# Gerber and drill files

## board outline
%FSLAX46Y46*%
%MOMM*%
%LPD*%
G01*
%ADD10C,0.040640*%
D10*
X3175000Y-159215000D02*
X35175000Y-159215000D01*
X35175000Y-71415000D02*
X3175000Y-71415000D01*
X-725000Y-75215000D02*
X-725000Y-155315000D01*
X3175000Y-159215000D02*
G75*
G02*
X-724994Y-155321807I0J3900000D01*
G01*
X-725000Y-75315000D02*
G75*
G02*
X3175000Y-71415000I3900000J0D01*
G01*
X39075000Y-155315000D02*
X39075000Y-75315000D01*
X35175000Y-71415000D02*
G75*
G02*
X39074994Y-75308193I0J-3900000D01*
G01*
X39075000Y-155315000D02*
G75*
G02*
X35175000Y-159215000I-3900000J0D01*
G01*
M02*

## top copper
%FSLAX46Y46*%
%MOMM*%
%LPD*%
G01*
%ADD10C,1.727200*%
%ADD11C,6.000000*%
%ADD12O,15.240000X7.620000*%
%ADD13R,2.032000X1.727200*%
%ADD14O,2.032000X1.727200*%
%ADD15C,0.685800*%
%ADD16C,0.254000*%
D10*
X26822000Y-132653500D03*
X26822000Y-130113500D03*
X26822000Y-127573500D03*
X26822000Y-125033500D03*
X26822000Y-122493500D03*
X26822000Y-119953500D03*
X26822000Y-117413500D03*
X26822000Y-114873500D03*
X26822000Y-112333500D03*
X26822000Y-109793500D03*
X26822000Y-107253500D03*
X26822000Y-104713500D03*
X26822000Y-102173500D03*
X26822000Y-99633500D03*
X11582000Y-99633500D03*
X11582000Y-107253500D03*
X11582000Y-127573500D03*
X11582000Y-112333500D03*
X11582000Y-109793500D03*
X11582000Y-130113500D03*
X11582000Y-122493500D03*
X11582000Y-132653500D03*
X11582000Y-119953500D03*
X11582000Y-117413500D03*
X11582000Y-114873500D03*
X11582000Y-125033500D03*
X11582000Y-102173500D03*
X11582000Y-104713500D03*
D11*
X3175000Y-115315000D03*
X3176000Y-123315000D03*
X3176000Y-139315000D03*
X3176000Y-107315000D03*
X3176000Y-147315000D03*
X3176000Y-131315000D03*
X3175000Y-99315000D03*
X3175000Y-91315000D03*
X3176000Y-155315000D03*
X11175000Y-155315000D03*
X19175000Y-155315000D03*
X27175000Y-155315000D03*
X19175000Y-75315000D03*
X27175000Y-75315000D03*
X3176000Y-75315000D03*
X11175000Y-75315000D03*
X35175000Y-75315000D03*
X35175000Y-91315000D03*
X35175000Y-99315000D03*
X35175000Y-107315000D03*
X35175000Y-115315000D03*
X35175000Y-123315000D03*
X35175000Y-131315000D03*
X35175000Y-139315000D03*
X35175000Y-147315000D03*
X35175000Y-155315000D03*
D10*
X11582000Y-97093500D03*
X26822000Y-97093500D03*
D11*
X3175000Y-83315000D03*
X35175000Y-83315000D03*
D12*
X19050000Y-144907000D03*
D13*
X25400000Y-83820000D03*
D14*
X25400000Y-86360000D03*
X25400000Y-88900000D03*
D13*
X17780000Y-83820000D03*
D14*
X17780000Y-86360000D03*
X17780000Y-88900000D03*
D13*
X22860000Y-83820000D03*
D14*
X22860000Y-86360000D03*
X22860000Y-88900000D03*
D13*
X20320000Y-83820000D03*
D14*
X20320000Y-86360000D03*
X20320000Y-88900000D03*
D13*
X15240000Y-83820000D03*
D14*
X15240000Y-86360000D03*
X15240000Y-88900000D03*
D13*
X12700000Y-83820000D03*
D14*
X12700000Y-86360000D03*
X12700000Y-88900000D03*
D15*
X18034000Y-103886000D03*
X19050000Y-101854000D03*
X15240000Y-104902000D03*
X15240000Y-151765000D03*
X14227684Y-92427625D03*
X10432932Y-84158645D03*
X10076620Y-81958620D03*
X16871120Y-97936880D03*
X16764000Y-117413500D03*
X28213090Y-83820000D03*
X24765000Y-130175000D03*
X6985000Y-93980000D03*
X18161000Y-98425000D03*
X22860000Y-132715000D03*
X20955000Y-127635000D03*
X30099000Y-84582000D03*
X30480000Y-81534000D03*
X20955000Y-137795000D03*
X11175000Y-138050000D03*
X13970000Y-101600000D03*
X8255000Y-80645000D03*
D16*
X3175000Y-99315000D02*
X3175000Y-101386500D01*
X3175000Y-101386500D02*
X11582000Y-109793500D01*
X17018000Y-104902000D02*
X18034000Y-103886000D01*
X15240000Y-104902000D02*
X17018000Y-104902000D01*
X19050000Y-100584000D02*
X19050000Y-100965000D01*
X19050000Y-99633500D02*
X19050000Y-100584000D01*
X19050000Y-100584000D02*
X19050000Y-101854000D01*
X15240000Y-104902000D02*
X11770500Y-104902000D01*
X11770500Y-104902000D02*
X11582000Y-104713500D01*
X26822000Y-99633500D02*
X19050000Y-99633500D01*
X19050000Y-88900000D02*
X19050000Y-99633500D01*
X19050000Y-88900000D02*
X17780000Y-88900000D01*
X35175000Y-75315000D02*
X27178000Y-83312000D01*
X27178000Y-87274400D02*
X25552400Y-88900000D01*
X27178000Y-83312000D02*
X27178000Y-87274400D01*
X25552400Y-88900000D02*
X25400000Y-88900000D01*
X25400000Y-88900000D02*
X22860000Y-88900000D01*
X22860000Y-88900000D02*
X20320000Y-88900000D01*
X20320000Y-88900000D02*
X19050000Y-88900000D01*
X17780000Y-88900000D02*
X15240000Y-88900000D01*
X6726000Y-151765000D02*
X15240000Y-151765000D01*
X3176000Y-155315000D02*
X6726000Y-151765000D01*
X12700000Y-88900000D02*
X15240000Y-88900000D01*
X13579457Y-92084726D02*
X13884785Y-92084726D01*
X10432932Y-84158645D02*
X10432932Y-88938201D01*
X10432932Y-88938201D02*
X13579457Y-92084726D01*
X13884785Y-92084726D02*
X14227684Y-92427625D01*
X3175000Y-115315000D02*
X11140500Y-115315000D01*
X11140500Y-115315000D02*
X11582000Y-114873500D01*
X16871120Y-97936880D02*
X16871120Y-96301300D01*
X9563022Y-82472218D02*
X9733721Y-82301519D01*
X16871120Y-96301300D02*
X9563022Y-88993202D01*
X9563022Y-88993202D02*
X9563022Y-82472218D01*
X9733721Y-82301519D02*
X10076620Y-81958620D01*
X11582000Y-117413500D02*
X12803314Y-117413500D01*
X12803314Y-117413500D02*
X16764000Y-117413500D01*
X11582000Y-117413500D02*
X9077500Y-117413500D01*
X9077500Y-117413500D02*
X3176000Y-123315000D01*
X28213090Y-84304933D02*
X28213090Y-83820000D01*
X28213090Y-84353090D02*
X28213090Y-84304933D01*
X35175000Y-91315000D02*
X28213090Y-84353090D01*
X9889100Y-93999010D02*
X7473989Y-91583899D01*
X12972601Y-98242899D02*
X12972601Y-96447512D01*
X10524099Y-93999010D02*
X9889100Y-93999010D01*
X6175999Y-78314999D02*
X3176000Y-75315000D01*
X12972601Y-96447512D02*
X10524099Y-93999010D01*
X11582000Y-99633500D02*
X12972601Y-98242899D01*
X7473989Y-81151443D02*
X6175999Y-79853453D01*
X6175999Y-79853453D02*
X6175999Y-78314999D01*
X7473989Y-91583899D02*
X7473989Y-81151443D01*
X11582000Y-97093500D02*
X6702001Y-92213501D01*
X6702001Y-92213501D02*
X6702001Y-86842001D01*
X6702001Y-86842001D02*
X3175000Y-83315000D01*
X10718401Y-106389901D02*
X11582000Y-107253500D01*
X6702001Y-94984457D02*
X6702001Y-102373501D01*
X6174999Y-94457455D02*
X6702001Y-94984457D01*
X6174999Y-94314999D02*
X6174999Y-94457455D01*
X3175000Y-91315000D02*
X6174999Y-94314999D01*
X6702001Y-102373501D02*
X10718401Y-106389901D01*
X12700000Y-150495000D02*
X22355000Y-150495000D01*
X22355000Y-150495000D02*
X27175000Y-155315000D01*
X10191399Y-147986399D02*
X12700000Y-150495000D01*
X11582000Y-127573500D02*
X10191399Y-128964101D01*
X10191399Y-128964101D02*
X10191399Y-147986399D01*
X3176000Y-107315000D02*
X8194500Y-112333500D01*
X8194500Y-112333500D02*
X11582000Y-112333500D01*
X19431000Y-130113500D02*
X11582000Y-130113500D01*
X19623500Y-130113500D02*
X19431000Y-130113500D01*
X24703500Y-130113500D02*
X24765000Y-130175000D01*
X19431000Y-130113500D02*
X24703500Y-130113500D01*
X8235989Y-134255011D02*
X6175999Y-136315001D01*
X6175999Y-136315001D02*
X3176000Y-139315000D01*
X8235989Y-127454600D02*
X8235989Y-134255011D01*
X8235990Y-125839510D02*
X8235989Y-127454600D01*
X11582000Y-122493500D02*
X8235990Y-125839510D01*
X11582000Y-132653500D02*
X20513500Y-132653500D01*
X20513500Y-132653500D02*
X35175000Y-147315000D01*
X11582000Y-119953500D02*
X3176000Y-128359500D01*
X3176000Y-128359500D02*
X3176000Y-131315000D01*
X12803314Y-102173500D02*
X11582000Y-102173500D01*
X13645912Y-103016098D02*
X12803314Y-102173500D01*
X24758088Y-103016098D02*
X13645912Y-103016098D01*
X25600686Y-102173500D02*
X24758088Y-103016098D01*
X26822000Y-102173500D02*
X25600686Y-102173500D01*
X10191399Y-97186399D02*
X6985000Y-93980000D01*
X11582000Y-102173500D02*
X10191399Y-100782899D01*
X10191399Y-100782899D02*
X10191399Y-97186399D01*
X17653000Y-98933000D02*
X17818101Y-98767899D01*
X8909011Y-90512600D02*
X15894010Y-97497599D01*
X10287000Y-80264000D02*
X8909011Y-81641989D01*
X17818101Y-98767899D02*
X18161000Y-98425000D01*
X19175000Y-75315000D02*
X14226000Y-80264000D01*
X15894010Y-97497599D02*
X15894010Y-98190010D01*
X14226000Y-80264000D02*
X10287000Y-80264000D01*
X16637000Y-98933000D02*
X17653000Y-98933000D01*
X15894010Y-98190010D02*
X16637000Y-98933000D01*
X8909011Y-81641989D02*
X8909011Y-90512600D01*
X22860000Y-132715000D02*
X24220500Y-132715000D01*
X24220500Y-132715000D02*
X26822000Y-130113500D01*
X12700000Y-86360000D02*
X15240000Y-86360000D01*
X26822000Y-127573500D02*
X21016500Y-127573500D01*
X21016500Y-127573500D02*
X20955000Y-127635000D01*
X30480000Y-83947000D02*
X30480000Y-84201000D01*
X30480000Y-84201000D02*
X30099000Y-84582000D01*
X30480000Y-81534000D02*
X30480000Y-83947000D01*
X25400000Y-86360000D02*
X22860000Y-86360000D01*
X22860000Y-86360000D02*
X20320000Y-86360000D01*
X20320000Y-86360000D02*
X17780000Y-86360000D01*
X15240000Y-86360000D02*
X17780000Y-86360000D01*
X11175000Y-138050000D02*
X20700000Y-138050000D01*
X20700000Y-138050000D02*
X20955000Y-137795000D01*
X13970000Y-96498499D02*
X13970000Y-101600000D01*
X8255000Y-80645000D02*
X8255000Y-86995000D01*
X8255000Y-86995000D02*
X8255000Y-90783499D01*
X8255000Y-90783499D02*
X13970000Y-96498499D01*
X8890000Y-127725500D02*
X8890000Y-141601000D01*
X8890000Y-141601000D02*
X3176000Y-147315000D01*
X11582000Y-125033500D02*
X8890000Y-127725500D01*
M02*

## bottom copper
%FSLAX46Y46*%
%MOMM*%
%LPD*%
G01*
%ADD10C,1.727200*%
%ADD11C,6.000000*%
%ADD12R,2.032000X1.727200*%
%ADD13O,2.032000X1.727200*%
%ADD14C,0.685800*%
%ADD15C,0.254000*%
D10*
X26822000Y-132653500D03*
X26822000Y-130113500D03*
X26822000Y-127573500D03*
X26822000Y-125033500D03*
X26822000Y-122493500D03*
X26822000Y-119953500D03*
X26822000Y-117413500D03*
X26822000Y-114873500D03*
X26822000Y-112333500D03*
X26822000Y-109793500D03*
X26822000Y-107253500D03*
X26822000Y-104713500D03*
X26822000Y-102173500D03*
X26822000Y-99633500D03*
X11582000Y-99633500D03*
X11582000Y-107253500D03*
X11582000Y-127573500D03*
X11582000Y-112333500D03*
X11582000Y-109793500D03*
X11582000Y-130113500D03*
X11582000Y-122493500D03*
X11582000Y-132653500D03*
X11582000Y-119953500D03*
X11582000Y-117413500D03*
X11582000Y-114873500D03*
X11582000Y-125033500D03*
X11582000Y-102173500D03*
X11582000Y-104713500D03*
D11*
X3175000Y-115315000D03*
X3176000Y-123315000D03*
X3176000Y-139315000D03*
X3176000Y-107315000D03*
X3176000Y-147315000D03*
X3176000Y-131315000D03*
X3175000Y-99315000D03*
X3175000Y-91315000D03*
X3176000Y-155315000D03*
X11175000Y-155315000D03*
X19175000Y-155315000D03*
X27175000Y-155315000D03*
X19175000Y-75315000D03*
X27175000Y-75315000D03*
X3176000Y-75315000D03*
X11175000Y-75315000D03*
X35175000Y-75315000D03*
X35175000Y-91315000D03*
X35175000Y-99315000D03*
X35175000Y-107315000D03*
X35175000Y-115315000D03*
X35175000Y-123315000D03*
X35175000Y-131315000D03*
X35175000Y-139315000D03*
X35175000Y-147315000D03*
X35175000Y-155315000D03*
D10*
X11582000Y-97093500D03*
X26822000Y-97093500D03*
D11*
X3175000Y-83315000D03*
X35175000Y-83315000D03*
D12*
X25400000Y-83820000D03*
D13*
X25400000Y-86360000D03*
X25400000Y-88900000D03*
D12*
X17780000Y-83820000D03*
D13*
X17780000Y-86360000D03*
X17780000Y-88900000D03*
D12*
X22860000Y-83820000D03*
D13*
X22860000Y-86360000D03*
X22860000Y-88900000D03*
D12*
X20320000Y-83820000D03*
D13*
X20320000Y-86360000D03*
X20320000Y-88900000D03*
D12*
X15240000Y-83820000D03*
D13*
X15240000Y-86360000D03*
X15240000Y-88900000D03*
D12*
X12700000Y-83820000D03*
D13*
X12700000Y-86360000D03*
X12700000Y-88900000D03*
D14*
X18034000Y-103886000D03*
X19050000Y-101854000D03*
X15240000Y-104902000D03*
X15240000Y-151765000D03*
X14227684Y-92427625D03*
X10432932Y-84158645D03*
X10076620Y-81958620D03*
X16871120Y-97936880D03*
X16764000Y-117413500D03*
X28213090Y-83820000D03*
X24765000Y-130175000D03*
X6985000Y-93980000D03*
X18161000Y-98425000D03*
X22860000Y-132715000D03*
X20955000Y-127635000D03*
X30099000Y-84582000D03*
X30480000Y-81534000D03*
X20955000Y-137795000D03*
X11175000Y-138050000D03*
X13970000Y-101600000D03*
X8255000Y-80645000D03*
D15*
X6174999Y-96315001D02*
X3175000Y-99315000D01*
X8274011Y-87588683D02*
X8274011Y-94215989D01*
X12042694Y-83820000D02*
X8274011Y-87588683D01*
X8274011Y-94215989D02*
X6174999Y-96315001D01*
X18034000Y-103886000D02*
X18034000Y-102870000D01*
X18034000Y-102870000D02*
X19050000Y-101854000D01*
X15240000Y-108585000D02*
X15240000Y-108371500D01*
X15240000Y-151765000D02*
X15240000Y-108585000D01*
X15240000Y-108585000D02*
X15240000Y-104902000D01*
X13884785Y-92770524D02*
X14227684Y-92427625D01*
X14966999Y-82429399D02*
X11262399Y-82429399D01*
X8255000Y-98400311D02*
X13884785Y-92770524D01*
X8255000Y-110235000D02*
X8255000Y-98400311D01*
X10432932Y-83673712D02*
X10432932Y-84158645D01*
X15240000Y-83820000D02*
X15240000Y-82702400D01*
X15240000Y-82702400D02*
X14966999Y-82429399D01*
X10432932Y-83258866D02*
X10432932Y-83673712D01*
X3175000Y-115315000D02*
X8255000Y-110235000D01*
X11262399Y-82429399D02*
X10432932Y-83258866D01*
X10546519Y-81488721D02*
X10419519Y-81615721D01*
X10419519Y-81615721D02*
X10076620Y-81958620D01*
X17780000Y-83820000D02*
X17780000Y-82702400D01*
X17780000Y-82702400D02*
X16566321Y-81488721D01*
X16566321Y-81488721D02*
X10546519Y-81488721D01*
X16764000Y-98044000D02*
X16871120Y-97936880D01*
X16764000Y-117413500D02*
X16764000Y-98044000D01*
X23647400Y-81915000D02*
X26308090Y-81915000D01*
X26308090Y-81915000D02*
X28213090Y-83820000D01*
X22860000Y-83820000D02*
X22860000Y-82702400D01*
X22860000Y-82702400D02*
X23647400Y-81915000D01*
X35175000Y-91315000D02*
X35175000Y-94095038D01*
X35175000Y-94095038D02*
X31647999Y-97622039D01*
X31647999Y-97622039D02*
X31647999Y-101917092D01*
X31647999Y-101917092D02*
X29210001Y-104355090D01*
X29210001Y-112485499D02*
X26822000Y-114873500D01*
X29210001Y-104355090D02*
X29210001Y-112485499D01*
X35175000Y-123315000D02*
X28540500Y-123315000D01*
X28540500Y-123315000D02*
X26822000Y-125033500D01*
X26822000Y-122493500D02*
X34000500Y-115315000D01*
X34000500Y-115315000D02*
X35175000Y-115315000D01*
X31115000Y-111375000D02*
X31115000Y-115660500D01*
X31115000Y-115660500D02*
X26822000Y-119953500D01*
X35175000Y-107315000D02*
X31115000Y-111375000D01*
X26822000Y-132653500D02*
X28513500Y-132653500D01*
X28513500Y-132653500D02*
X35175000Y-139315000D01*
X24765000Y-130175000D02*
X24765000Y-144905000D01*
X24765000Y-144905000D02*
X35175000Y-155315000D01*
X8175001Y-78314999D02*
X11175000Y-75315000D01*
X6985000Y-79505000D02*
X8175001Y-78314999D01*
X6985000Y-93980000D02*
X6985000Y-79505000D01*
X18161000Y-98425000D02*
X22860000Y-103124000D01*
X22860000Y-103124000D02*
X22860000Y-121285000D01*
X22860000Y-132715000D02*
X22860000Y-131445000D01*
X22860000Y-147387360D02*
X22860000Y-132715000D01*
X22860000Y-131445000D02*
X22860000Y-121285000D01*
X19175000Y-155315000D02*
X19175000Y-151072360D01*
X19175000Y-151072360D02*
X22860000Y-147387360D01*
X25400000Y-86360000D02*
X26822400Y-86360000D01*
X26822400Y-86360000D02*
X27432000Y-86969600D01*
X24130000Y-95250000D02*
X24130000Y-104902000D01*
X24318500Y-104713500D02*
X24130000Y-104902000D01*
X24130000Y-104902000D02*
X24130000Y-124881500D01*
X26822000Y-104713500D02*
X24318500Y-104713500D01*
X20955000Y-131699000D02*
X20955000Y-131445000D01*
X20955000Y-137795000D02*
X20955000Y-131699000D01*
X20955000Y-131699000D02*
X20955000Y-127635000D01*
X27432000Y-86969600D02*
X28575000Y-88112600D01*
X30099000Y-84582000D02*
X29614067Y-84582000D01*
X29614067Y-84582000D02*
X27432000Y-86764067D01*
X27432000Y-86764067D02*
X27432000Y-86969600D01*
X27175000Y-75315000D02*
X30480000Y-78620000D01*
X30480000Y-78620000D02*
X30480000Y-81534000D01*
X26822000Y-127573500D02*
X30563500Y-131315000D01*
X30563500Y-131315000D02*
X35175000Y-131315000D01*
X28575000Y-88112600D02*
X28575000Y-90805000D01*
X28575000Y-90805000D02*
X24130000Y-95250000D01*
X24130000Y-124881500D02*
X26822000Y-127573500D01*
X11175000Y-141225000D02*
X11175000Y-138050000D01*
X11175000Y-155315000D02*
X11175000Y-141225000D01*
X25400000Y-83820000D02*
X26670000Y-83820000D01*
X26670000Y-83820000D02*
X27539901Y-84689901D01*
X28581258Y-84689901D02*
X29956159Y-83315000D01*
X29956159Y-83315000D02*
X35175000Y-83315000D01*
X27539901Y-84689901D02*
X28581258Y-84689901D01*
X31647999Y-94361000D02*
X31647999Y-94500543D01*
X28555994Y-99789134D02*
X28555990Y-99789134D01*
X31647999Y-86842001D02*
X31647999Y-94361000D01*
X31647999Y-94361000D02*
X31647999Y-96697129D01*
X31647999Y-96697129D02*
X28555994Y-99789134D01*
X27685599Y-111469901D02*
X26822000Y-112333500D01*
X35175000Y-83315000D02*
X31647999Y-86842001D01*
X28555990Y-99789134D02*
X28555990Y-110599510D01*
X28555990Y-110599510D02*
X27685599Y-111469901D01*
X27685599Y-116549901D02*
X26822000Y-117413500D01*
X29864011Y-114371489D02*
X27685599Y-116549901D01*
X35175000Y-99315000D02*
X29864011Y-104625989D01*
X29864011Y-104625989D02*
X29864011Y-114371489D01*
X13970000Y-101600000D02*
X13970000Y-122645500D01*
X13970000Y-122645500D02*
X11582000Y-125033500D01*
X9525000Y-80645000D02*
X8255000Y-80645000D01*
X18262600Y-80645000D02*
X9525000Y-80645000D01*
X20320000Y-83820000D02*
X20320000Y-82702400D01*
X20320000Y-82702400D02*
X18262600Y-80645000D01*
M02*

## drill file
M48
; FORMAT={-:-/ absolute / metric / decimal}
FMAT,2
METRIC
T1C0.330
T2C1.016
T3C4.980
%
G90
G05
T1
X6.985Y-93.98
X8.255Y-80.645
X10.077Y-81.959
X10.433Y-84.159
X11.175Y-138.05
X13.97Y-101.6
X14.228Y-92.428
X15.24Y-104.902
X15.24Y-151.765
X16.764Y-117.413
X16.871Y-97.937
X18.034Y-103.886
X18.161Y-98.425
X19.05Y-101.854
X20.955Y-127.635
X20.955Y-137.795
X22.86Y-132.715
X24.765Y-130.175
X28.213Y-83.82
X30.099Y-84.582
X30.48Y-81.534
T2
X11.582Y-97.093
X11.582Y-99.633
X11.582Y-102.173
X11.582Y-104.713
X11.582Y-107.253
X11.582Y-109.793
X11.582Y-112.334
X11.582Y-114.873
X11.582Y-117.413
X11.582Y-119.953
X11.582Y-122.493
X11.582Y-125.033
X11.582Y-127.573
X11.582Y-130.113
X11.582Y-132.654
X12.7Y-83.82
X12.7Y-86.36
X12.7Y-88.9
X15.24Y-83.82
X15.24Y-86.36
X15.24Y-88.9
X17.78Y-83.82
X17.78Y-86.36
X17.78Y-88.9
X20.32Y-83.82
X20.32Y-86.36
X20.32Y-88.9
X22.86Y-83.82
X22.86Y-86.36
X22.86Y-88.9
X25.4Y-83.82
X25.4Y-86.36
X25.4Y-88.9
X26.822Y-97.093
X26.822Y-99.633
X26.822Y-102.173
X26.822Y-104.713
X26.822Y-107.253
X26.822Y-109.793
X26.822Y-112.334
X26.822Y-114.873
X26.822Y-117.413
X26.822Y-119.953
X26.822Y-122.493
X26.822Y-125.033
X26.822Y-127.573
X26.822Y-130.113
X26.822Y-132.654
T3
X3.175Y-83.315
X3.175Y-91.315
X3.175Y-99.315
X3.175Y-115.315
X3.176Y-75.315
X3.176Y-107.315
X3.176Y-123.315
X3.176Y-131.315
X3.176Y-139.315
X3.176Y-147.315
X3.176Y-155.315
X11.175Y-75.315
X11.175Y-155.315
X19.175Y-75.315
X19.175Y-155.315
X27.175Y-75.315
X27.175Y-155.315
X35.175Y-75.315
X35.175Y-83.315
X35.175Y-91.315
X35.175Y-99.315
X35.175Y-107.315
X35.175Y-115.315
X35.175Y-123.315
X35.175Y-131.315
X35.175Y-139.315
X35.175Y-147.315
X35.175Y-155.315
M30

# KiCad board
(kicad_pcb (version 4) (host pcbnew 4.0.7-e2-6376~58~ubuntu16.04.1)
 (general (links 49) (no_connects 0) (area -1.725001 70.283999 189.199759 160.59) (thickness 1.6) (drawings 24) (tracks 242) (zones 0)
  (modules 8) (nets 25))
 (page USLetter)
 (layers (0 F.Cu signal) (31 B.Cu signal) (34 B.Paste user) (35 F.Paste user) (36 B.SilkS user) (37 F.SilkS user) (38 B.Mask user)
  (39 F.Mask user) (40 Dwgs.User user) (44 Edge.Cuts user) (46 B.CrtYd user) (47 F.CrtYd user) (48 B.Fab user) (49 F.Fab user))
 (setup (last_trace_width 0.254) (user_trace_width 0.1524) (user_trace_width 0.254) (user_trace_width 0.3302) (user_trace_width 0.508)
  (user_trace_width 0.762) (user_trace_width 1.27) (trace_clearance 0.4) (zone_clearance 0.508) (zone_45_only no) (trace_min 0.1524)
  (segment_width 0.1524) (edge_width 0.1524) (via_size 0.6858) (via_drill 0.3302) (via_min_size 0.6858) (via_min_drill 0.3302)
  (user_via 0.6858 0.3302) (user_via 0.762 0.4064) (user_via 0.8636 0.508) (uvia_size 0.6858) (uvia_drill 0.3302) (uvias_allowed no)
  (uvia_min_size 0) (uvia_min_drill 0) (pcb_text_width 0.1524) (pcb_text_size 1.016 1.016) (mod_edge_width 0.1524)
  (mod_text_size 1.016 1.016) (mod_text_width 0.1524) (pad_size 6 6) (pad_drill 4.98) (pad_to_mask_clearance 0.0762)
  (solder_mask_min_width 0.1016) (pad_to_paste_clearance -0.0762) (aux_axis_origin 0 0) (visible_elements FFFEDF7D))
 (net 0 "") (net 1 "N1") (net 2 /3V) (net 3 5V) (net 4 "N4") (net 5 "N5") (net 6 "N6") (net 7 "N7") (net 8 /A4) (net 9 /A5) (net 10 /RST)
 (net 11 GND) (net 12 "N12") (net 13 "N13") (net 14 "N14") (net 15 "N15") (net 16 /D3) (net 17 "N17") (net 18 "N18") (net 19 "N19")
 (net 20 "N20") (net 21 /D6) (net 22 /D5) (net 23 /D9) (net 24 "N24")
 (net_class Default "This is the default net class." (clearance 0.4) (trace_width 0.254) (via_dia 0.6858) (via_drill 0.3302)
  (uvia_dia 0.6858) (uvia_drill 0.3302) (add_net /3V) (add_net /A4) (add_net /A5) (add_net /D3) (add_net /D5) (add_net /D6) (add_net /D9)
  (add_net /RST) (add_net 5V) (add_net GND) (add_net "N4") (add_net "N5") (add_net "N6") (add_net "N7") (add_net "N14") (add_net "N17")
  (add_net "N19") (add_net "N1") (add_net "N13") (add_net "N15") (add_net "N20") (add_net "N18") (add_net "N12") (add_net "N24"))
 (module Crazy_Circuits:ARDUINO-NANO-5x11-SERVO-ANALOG (layer F.Cu) (at 3.175 107.315)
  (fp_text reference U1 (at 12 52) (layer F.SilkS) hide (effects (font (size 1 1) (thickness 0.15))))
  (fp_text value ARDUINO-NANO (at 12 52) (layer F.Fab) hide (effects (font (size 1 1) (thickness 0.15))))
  (fp_line (start 0 51.9) (end 32 51.9) (layer Edge.Cuts) (width 0.04064))
  (fp_line (start 32 -35.9) (end 0 -35.9) (layer Edge.Cuts) (width 0.04064))
  (fp_line (start -3.9 -32.1) (end -3.9 48) (layer Edge.Cuts) (width 0.04064))
  (fp_arc (start 0 48) (end 0 51.9) (angle 89.9) (layer Edge.Cuts) (width 0.04064))
  (fp_arc (start 0 -32) (end -3.9 -32) (angle 90) (layer Edge.Cuts) (width 0.04064))
  (fp_line (start 35.9 48) (end 35.9 -32) (layer Edge.Cuts) (width 0.04064))
  (fp_arc (start 32 -32) (end 32 -35.9) (angle 89.9) (layer Edge.Cuts) (width 0.04064))
  (fp_arc (start 32 48) (end 35.9 48) (angle 90) (layer Edge.Cuts) (width 0.04064))
  (pad D13 thru_hole circle (at 23.647 25.3385 180) (size 1.7272 1.7272) (drill 1.016) (layers *.Cu *.Mask F.SilkS) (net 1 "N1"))
  (pad 3V thru_hole circle (at 23.647 22.7985 180) (size 1.7272 1.7272) (drill 1.016) (layers *.Cu *.Mask F.SilkS) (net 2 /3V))
  (pad REF thru_hole circle (at 23.647 20.2585 180) (size 1.7272 1.7272) (drill 1.016) (layers *.Cu *.Mask F.SilkS) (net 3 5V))
  (pad A0 thru_hole circle (at 23.647 17.7185 180) (size 1.7272 1.7272) (drill 1.016) (layers *.Cu *.Mask F.SilkS) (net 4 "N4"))
  (pad A1 thru_hole circle (at 23.647 15.1785 180) (size 1.7272 1.7272) (drill 1.016) (layers *.Cu *.Mask F.SilkS) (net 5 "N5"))
  (pad A2 thru_hole circle (at 23.647 12.6385 180) (size 1.7272 1.7272) (drill 1.016) (layers *.Cu *.Mask F.SilkS) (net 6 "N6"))
  (pad A3 thru_hole circle (at 23.647 10.0985 180) (size 1.7272 1.7272) (drill 1.016) (layers *.Cu *.Mask F.SilkS) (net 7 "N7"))
  (pad A4 thru_hole circle (at 23.647 7.5585 180) (size 1.7272 1.7272) (drill 1.016) (layers *.Cu *.Mask F.SilkS) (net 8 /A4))
  (pad A5 thru_hole circle (at 23.647 5.0185 180) (size 1.7272 1.7272) (drill 1.016) (layers *.Cu *.Mask F.SilkS) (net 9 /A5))
  (pad A6 thru_hole circle (at 23.647 2.4785 180) (size 1.7272 1.7272) (drill 1.016) (layers *.Cu *.Mask F.SilkS))
  (pad A7 thru_hole circle (at 23.647 -0.0615 180) (size 1.7272 1.7272) (drill 1.016) (layers *.Cu *.Mask F.SilkS))
  (pad 5V thru_hole circle (at 23.647 -2.6015 180) (size 1.7272 1.7272) (drill 1.016) (layers *.Cu *.Mask F.SilkS) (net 3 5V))
  (pad RST thru_hole circle (at 23.647 -5.1415 180) (size 1.7272 1.7272) (drill 1.016) (layers *.Cu *.Mask F.SilkS) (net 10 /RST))
  (pad GND thru_hole circle (at 23.647 -7.6815 180) (size 1.7272 1.7272) (drill 1.016) (layers *.Cu *.Mask F.SilkS) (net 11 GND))
  (pad RX0 thru_hole circle (at 8.407 -7.6815 180) (size 1.7272 1.7272) (drill 1.016) (layers *.Cu *.Mask F.SilkS) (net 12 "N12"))
  (pad D2 thru_hole circle (at 8.407 -0.0615 180) (size 1.7272 1.7272) (drill 1.016) (layers *.Cu *.Mask F.SilkS) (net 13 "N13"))
  (pad D10 thru_hole circle (at 8.407 20.2585 180) (size 1.7272 1.7272) (drill 1.016) (layers *.Cu *.Mask F.SilkS) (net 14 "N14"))
  (pad D4 thru_hole circle (at 8.407 5.0185 180) (size 1.7272 1.7272) (drill 1.016) (layers *.Cu *.Mask F.SilkS) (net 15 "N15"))
  (pad D3 thru_hole circle (at 8.407 2.4785 180) (size 1.7272 1.7272) (drill 1.016) (layers *.Cu *.Mask F.SilkS) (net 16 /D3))
  (pad D11 thru_hole circle (at 8.407 22.7985 180) (size 1.7272 1.7272) (drill 1.016) (layers *.Cu *.Mask F.SilkS) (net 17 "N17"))
  (pad D8 thru_hole circle (at 8.407 15.1785 180) (size 1.7272 1.7272) (drill 1.016) (layers *.Cu *.Mask F.SilkS) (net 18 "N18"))
  (pad D12 thru_hole circle (at 8.407 25.3385 180) (size 1.7272 1.7272) (drill 1.016) (layers *.Cu *.Mask F.SilkS) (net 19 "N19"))
  (pad D7 thru_hole circle (at 8.407 12.6385 180) (size 1.7272 1.7272) (drill 1.016) (layers *.Cu *.Mask F.SilkS) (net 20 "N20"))
  (pad D6 thru_hole circle (at 8.407 10.0985 180) (size 1.7272 1.7272) (drill 1.016) (layers *.Cu *.Mask F.SilkS) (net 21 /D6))
  (pad D5 thru_hole circle (at 8.407 7.5585 180) (size 1.7272 1.7272) (drill 1.016) (layers *.Cu *.Mask F.SilkS) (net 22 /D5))
  (pad D9 thru_hole circle (at 8.407 17.7185 180) (size 1.7272 1.7272) (drill 1.016) (layers *.Cu *.Mask F.SilkS) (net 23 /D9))
  (pad RST thru_hole circle (at 8.407 -5.1415 180) (size 1.7272 1.7272) (drill 1.016) (layers *.Cu *.Mask F.SilkS) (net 10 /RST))
  (pad GND thru_hole circle (at 8.407 -2.6015 180) (size 1.7272 1.7272) (drill 1.016) (layers *.Cu *.Mask F.SilkS) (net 11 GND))
  (pad D5 thru_hole circle (at 0 8 90) (size 6 6) (drill 4.98) (layers *.Cu *.Mask) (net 22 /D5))
  (pad D6 thru_hole circle (at 0.001 16 90) (size 6 6) (drill 4.98) (layers *.Cu *.Mask) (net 21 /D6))
  (pad D8 thru_hole circle (at 0.001 32 90) (size 6 6) (drill 4.98) (layers *.Cu *.Mask) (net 18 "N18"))
  (pad D4 thru_hole circle (at 0.001 0 90) (size 6 6) (drill 4.98) (layers *.Cu *.Mask) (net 15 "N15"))
  (pad D9 thru_hole circle (at 0.001 40 90) (size 6 6) (drill 4.98) (layers *.Cu *.Mask) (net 23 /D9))
  (pad D7 thru_hole circle (at 0.001 24 90) (size 6 6) (drill 4.98) (layers *.Cu *.Mask) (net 20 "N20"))
  (pad D3 thru_hole circle (at 0 -8 90) (size 6 6) (drill 4.98) (layers *.Cu *.Mask) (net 16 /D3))
  (pad D2 thru_hole circle (at 0 -16 90) (size 6 6) (drill 4.98) (layers *.Cu *.Mask) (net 13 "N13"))
  (pad GND thru_hole circle (at 0.001 48 90) (size 6 6) (drill 4.98) (layers *.Cu *.Mask) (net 11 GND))
  (pad 5V thru_hole circle (at 8 48 90) (size 6 6) (drill 4.98) (layers *.Cu *.Mask) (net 3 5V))
  (pad 3V thru_hole circle (at 16 48 90) (size 6 6) (drill 4.98) (layers *.Cu *.Mask) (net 2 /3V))
  (pad D10 thru_hole circle (at 24 48 90) (size 6 6) (drill 4.98) (layers *.Cu *.Mask) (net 14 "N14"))
  (pad 3V thru_hole circle (at 16 -32 90) (size 6 6) (drill 4.98) (layers *.Cu *.Mask) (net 2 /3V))
  (pad 5V thru_hole circle (at 24 -32 90) (size 6 6) (drill 4.98) (layers *.Cu *.Mask) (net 3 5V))
  (pad RX0 thru_hole circle (at 0.001 -32 90) (size 6 6) (drill 4.98) (layers *.Cu *.Mask) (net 12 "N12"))
  (pad RST thru_hole circle (at 8 -32 90) (size 6 6) (drill 4.98) (layers *.Cu *.Mask) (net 10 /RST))
  (pad GND thru_hole circle (at 32 -32 90) (size 6 6) (drill 4.98) (layers *.Cu *.Mask) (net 11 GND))
  (pad A4 thru_hole circle (at 32 -16 90) (size 6 6) (drill 4.98) (layers *.Cu *.Mask) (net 8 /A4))
  (pad A3 thru_hole circle (at 32 -8 90) (size 6 6) (drill 4.98) (layers *.Cu *.Mask) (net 7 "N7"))
  (pad A2 thru_hole circle (at 32 0 90) (size 6 6) (drill 4.98) (layers *.Cu *.Mask) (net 6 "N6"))
  (pad A1 thru_hole circle (at 32 8 90) (size 6 6) (drill 4.98) (layers *.Cu *.Mask) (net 5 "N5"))
  (pad A0 thru_hole circle (at 32 16 90) (size 6 6) (drill 4.98) (layers *.Cu *.Mask) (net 4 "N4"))
  (pad REF thru_hole circle (at 32 24 90) (size 6 6) (drill 4.98) (layers *.Cu *.Mask) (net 3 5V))
  (pad D13 thru_hole circle (at 32 32 90) (size 6 6) (drill 4.98) (layers *.Cu *.Mask) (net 1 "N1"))
  (pad D12 thru_hole circle (at 32 40 90) (size 6 6) (drill 4.98) (layers *.Cu *.Mask) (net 19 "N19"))
  (pad D11 thru_hole circle (at 32 48 90) (size 6 6) (drill 4.98) (layers *.Cu *.Mask) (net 17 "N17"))
  (pad TX1 thru_hole circle (at 8.407 -10.2215 180) (size 1.7272 1.7272) (drill 1.016) (layers *.Cu *.Mask F.SilkS) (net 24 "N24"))
  (pad VIN thru_hole circle (at 23.647 -10.2215 180) (size 1.7272 1.7272) (drill 1.016) (layers *.Cu *.Mask F.SilkS))
  (pad TX1 thru_hole circle (at 0 -24 90) (size 6 6) (drill 4.98) (layers *.Cu *.Mask) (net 24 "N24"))
  (pad A5 thru_hole circle (at 32 -24 90) (size 6 6) (drill 4.98) (layers *.Cu *.Mask) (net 9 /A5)))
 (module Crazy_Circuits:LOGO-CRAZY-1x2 (layer F.Cu) (at 19.05 148.844)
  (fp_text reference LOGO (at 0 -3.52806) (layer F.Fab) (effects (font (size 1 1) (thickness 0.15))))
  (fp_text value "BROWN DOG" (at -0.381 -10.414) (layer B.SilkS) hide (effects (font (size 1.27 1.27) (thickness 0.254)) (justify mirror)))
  (pad BG smd oval (at 0 -3.937) (size 15.24 7.62) (layers F.Cu)))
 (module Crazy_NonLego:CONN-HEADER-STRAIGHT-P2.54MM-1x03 (layer F.Cu) (at 25.4 83.82)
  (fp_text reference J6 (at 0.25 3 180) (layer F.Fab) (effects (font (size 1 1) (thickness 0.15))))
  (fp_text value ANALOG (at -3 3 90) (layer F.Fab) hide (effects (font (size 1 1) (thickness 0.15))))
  (pad 1 thru_hole rect (at 0 0) (size 2.032 1.7272) (drill 1.016) (layers *.Cu *.Mask F.SilkS) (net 9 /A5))
  (pad 2 thru_hole oval (at 0 2.54) (size 2.032 1.7272) (drill 1.016) (layers *.Cu *.Mask F.SilkS) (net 3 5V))
  (pad 3 thru_hole oval (at 0 5.08) (size 2.032 1.7272) (drill 1.016) (layers *.Cu *.Mask F.SilkS) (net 11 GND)))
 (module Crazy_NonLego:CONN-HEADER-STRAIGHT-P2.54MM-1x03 (layer F.Cu) (at 17.78 83.82)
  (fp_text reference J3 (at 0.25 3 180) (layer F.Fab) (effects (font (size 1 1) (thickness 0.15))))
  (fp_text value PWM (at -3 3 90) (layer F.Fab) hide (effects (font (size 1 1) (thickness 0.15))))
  (pad 1 thru_hole rect (at 0 0) (size 2.032 1.7272) (drill 1.016) (layers *.Cu *.Mask F.SilkS) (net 21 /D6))
  (pad 2 thru_hole oval (at 0 2.54) (size 2.032 1.7272) (drill 1.016) (layers *.Cu *.Mask F.SilkS) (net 3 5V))
  (pad 3 thru_hole oval (at 0 5.08) (size 2.032 1.7272) (drill 1.016) (layers *.Cu *.Mask F.SilkS) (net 11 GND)))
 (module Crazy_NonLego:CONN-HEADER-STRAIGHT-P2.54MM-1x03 (layer F.Cu) (at 22.86 83.82)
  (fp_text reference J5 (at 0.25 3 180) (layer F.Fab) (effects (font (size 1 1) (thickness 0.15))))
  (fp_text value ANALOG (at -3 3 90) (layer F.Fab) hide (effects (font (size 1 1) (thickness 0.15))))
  (pad 1 thru_hole rect (at 0 0) (size 2.032 1.7272) (drill 1.016) (layers *.Cu *.Mask F.SilkS) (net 8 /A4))
  (pad 2 thru_hole oval (at 0 2.54) (size 2.032 1.7272) (drill 1.016) (layers *.Cu *.Mask F.SilkS) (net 3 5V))
  (pad 3 thru_hole oval (at 0 5.08) (size 2.032 1.7272) (drill 1.016) (layers *.Cu *.Mask F.SilkS) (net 11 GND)))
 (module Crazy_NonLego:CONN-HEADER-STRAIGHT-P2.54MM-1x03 (layer F.Cu) (at 20.32 83.82)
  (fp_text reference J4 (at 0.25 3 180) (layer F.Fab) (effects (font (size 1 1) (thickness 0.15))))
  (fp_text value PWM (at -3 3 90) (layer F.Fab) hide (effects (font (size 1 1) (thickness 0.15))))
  (pad 1 thru_hole rect (at 0 0) (size 2.032 1.7272) (drill 1.016) (layers *.Cu *.Mask F.SilkS) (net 23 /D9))
  (pad 2 thru_hole oval (at 0 2.54) (size 2.032 1.7272) (drill 1.016) (layers *.Cu *.Mask F.SilkS) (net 3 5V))
  (pad 3 thru_hole oval (at 0 5.08) (size 2.032 1.7272) (drill 1.016) (layers *.Cu *.Mask F.SilkS) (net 11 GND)))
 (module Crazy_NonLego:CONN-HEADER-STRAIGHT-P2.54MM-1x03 (layer F.Cu) (at 15.24 83.82)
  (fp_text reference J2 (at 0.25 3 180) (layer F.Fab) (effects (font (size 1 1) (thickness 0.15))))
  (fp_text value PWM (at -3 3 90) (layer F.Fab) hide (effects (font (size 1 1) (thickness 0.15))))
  (pad 1 thru_hole rect (at 0 0) (size 2.032 1.7272) (drill 1.016) (layers *.Cu *.Mask F.SilkS) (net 22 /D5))
  (pad 2 thru_hole oval (at 0 2.54) (size 2.032 1.7272) (drill 1.016) (layers *.Cu *.Mask F.SilkS) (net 3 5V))
  (pad 3 thru_hole oval (at 0 5.08) (size 2.032 1.7272) (drill 1.016) (layers *.Cu *.Mask F.SilkS) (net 11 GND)))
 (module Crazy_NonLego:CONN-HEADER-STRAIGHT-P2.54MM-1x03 (layer F.Cu) (at 12.7 83.82)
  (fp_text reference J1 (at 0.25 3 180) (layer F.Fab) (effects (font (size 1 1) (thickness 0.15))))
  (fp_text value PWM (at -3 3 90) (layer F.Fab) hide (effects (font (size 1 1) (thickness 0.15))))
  (pad 1 thru_hole rect (at 0 0) (size 2.032 1.7272) (drill 1.016) (layers *.Cu *.Mask F.SilkS) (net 16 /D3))
  (pad 2 thru_hole oval (at 0 2.54) (size 2.032 1.7272) (drill 1.016) (layers *.Cu *.Mask F.SilkS) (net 3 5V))
  (pad 3 thru_hole oval (at 0 5.08) (size 2.032 1.7272) (drill 1.016) (layers *.Cu *.Mask F.SilkS) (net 11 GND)))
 (segment (start 6.174999 96.315001) (end 3.175 99.315) (width 0.254) (layer B.Cu) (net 16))
 (segment (start 8.274011 87.588683) (end 8.274011 94.215989) (width 0.254) (layer B.Cu) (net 16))
 (segment (start 12.042694 83.82) (end 8.274011 87.588683) (width 0.254) (layer B.Cu) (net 16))
 (segment (start 8.274011 94.215989) (end 6.174999 96.315001) (width 0.254) (layer B.Cu) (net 16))
 (segment (start 3.175 99.315) (end 3.175 101.3865) (width 0.254) (layer F.Cu) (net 16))
 (segment (start 3.175 101.3865) (end 11.582 109.7935) (width 0.254) (layer F.Cu) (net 16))
 (segment (start 18.034 103.886) (end 18.034 102.87) (width 0.254) (layer B.Cu) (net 11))
 (segment (start 18.034 102.87) (end 19.05 101.854) (width 0.254) (layer B.Cu) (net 11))
 (segment (start 17.018 104.902) (end 18.034 103.886) (width 0.254) (layer F.Cu) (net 11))
 (via (at 18.034 103.886) (size 0.6858) (drill 0.3302) (layers F.Cu B.Cu) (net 11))
 (segment (start 15.24 104.902) (end 17.018 104.902) (width 0.254) (layer F.Cu) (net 11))
 (segment (start 19.05 100.584) (end 19.05 100.965) (width 0.254) (layer F.Cu) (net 11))
 (segment (start 19.05 99.6335) (end 19.05 100.584) (width 0.254) (layer F.Cu) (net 11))
 (segment (start 19.05 100.584) (end 19.05 101.854) (width 0.254) (layer F.Cu) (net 11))
 (via (at 19.05 101.854) (size 0.6858) (drill 0.3302) (layers F.Cu B.Cu) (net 11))
 (segment (start 15.24 108.585) (end 15.24 108.3715) (width 0.254) (layer B.Cu) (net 11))
 (segment (start 15.24 151.765) (end 15.24 108.585) (width 0.254) (layer B.Cu) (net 11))
 (segment (start 15.24 104.902) (end 11.7705 104.902) (width 0.254) (layer F.Cu) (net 11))
 (segment (start 15.24 108.585) (end 15.24 104.902) (width 0.254) (layer B.Cu) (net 11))
 (via (at 15.24 104.902) (size 0.6858) (drill 0.3302) (layers F.Cu B.Cu) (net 11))
 (segment (start 11.7705 104.902) (end 11.582 104.7135) (width 0.254) (layer F.Cu) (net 11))
 (segment (start 26.822 99.6335) (end 19.05 99.6335) (width 0.254) (layer F.Cu) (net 11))
 (segment (start 19.05 88.9) (end 19.05 99.6335) (width 0.254) (layer F.Cu) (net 11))
 (segment (start 19.05 88.9) (end 17.78 88.9) (width 0.254) (layer F.Cu) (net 11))
 (segment (start 35.175 75.315) (end 27.178 83.312) (width 0.254) (layer F.Cu) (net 11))
 (segment (start 27.178 87.2744) (end 25.5524 88.9) (width 0.254) (layer F.Cu) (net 11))
 (segment (start 27.178 83.312) (end 27.178 87.2744) (width 0.254) (layer F.Cu) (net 11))
 (segment (start 25.5524 88.9) (end 25.4 88.9) (width 0.254) (layer F.Cu) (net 11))
 (segment (start 25.4 88.9) (end 22.86 88.9) (width 0.254) (layer F.Cu) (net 11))
 (segment (start 22.86 88.9) (end 20.32 88.9) (width 0.254) (layer F.Cu) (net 11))
 (segment (start 20.32 88.9) (end 19.05 88.9) (width 0.254) (layer F.Cu) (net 11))
 (segment (start 17.78 88.9) (end 15.24 88.9) (width 0.254) (layer F.Cu) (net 11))
 (segment (start 6.726 151.765) (end 15.24 151.765) (width 0.254) (layer F.Cu) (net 11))
 (via (at 15.24 151.765) (size 0.6858) (drill 0.3302) (layers F.Cu B.Cu) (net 11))
 (segment (start 3.176 155.315) (end 6.726 151.765) (width 0.254) (layer F.Cu) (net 11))
 (segment (start 12.7 88.9) (end 15.24 88.9) (width 0.254) (layer F.Cu) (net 11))
 (segment (start 13.884785 92.770524) (end 14.227684 92.427625) (width 0.254) (layer B.Cu) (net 22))
 (segment (start 13.579457 92.084726) (end 13.884785 92.084726) (width 0.254) (layer F.Cu) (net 22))
 (segment (start 14.966999 82.429399) (end 11.262399 82.429399) (width 0.254) (layer B.Cu) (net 22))
 (segment (start 8.255 98.400311) (end 13.884785 92.770524) (width 0.254) (layer B.Cu) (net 22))
 (segment (start 8.255 110.235) (end 8.255 98.400311) (width 0.254) (layer B.Cu) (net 22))
 (segment (start 10.432932 83.673712) (end 10.432932 84.158645) (width 0.254) (layer B.Cu) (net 22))
 (segment (start 15.24 83.82) (end 15.24 82.7024) (width 0.254) (layer B.Cu) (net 22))
 (segment (start 10.432932 84.158645) (end 10.432932 88.938201) (width 0.254) (layer F.Cu) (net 22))
 (segment (start 15.24 82.7024) (end 14.966999 82.429399) (width 0.254) (layer B.Cu) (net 22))
 (segment (start 10.432932 88.938201) (end 13.579457 92.084726) (width 0.254) (layer F.Cu) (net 22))
 (segment (start 10.432932 83.258866) (end 10.432932 83.673712) (width 0.254) (layer B.Cu) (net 22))
 (segment (start 3.175 115.315) (end 8.255 110.235) (width 0.254) (layer B.Cu) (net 22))
 (segment (start 13.884785 92.084726) (end 14.227684 92.427625) (width 0.254) (layer F.Cu) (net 22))
 (via (at 14.227684 92.427625) (size 0.6858) (drill 0.3302) (layers F.Cu B.Cu) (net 22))
 (segment (start 11.262399 82.429399) (end 10.432932 83.258866) (width 0.254) (layer B.Cu) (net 22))
 (via (at 10.432932 84.158645) (size 0.6858) (drill 0.3302) (layers F.Cu B.Cu) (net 22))
 (segment (start 3.175 115.315) (end 11.1405 115.315) (width 0.254) (layer F.Cu) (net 22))
 (segment (start 11.1405 115.315) (end 11.582 114.8735) (width 0.254) (layer F.Cu) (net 22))
 (segment (start 16.87112 97.93688) (end 16.87112 96.3013) (width 0.254) (layer F.Cu) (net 21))
 (segment (start 9.563022 82.472218) (end 9.733721 82.301519) (width 0.254) (layer F.Cu) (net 21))
 (segment (start 16.87112 96.3013) (end 9.563022 88.993202) (width 0.254) (layer F.Cu) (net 21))
 (segment (start 9.563022 88.993202) (end 9.563022 82.472218) (width 0.254) (layer F.Cu) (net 21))
 (segment (start 9.733721 82.301519) (end 10.07662 81.95862) (width 0.254) (layer F.Cu) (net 21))
 (via (at 10.07662 81.95862) (size 0.6858) (drill 0.3302) (layers F.Cu B.Cu) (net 21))
 (segment (start 10.546519 81.488721) (end 10.419519 81.615721) (width 0.254) (layer B.Cu) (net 21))
 (segment (start 10.419519 81.615721) (end 10.07662 81.95862) (width 0.254) (layer B.Cu) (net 21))
 (segment (start 17.78 83.82) (end 17.78 82.7024) (width 0.254) (layer B.Cu) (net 21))
 (segment (start 17.78 82.7024) (end 16.566321 81.488721) (width 0.254) (layer B.Cu) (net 21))
 (segment (start 16.566321 81.488721) (end 10.546519 81.488721) (width 0.254) (layer B.Cu) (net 21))
 (segment (start 16.764 98.044) (end 16.87112 97.93688) (width 0.254) (layer B.Cu) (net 21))
 (via (at 16.87112 97.93688) (size 0.6858) (drill 0.3302) (layers F.Cu B.Cu) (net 21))
 (segment (start 16.764 117.4135) (end 16.764 98.044) (width 0.254) (layer B.Cu) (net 21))
 (segment (start 11.582 117.4135) (end 12.803314 117.4135) (width 0.254) (layer F.Cu) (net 21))
 (segment (start 12.803314 117.4135) (end 16.764 117.4135) (width 0.254) (layer F.Cu) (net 21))
 (via (at 16.764 117.4135) (size 0.6858) (drill 0.3302) (layers F.Cu B.Cu) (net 21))
 (segment (start 11.582 117.4135) (end 9.0775 117.4135) (width 0.254) (layer F.Cu) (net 21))
 (segment (start 9.0775 117.4135) (end 3.176 123.315) (width 0.254) (layer F.Cu) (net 21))
 (segment (start 23.6474 81.915) (end 26.30809 81.915) (width 0.254) (layer B.Cu) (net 8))
 (segment (start 26.30809 81.915) (end 28.21309 83.82) (width 0.254) (layer B.Cu) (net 8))
 (segment (start 22.86 83.82) (end 22.86 82.7024) (width 0.254) (layer B.Cu) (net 8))
 (segment (start 22.86 82.7024) (end 23.6474 81.915) (width 0.254) (layer B.Cu) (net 8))
 (segment (start 28.21309 84.304933) (end 28.21309 83.82) (width 0.254) (layer F.Cu) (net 8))
 (segment (start 28.21309 84.35309) (end 28.21309 84.304933) (width 0.254) (layer F.Cu) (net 8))
 (segment (start 35.175 91.315) (end 28.21309 84.35309) (width 0.254) (layer F.Cu) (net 8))
 (via (at 28.21309 83.82) (size 0.6858) (drill 0.3302) (layers F.Cu B.Cu) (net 8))
 (segment (start 35.175 91.315) (end 35.175 94.095038) (width 0.254) (layer B.Cu) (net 8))
 (segment (start 35.175 94.095038) (end 31.647999 97.622039) (width 0.254) (layer B.Cu) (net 8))
 (segment (start 31.647999 97.622039) (end 31.647999 101.917092) (width 0.254) (layer B.Cu) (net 8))
 (segment (start 31.647999 101.917092) (end 29.210001 104.35509) (width 0.254) (layer B.Cu) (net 8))
 (segment (start 29.210001 112.485499) (end 26.822 114.8735) (width 0.254) (layer B.Cu) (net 8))
 (segment (start 29.210001 104.35509) (end 29.210001 112.485499) (width 0.254) (layer B.Cu) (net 8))
 (segment (start 35.175 123.315) (end 28.5405 123.315) (width 0.254) (layer B.Cu) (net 4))
 (segment (start 28.5405 123.315) (end 26.822 125.0335) (width 0.254) (layer B.Cu) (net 4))
 (segment (start 26.822 122.4935) (end 34.0005 115.315) (width 0.254) (layer B.Cu) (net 5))
 (segment (start 34.0005 115.315) (end 35.175 115.315) (width 0.254) (layer B.Cu) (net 5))
 (segment (start 31.115 111.375) (end 31.115 115.6605) (width 0.254) (layer B.Cu) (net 6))
 (segment (start 31.115 115.6605) (end 26.822 119.9535) (width 0.254) (layer B.Cu) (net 6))
 (segment (start 35.175 107.315) (end 31.115 111.375) (width 0.254) (layer B.Cu) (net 6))
 (segment (start 9.8891 93.99901) (end 7.473989 91.583899) (width 0.254) (layer F.Cu) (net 12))
 (segment (start 12.972601 98.242899) (end 12.972601 96.447512) (width 0.254) (layer F.Cu) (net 12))
 (segment (start 10.524099 93.99901) (end 9.8891 93.99901) (width 0.254) (layer F.Cu) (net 12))
 (segment (start 6.175999 78.314999) (end 3.176 75.315) (width 0.254) (layer F.Cu) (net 12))
 (segment (start 12.972601 96.447512) (end 10.524099 93.99901) (width 0.254) (layer F.Cu) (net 12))
 (segment (start 11.582 99.6335) (end 12.972601 98.242899) (width 0.254) (layer F.Cu) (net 12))
 (segment (start 7.473989 81.151443) (end 6.175999 79.853453) (width 0.254) (layer F.Cu) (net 12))
 (segment (start 6.175999 79.853453) (end 6.175999 78.314999) (width 0.254) (layer F.Cu) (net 12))
 (segment (start 7.473989 91.583899) (end 7.473989 81.151443) (width 0.254) (layer F.Cu) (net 12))
 (segment (start 11.582 97.0935) (end 6.702001 92.213501) (width 0.254) (layer F.Cu) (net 24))
 (segment (start 6.702001 92.213501) (end 6.702001 86.842001) (width 0.254) (layer F.Cu) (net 24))
 (segment (start 6.702001 86.842001) (end 3.175 83.315) (width 0.254) (layer F.Cu) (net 24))
 (segment (start 26.822 132.6535) (end 28.5135 132.6535) (width 0.254) (layer B.Cu) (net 1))
 (segment (start 28.5135 132.6535) (end 35.175 139.315) (width 0.254) (layer B.Cu) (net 1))
 (segment (start 10.718401 106.389901) (end 11.582 107.2535) (width 0.254) (layer F.Cu) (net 13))
 (segment (start 6.702001 94.984457) (end 6.702001 102.373501) (width 0.254) (layer F.Cu) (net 13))
 (segment (start 6.174999 94.457455) (end 6.702001 94.984457) (width 0.254) (layer F.Cu) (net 13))
 (segment (start 6.174999 94.314999) (end 6.174999 94.457455) (width 0.254) (layer F.Cu) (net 13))
 (segment (start 3.175 91.315) (end 6.174999 94.314999) (width 0.254) (layer F.Cu) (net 13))
 (segment (start 6.702001 102.373501) (end 10.718401 106.389901) (width 0.254) (layer F.Cu) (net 13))
 (segment (start 12.7 150.495) (end 22.355 150.495) (width 0.254) (layer F.Cu) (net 14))
 (segment (start 22.355 150.495) (end 27.175 155.315) (width 0.254) (layer F.Cu) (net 14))
 (segment (start 10.191399 147.986399) (end 12.7 150.495) (width 0.254) (layer F.Cu) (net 14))
 (segment (start 11.582 127.5735) (end 10.191399 128.964101) (width 0.254) (layer F.Cu) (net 14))
 (segment (start 10.191399 128.964101) (end 10.191399 147.986399) (width 0.254) (layer F.Cu) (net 14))
 (segment (start 3.176 107.315) (end 8.1945 112.3335) (width 0.254) (layer F.Cu) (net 15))
 (segment (start 8.1945 112.3335) (end 11.582 112.3335) (width 0.254) (layer F.Cu) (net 15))
 (segment (start 19.431 130.1135) (end 11.582 130.1135) (width 0.254) (layer F.Cu) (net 17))
 (segment (start 19.6235 130.1135) (end 19.431 130.1135) (width 0.254) (layer F.Cu) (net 17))
 (segment (start 24.7035 130.1135) (end 24.765 130.175) (width 0.254) (layer F.Cu) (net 17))
 (via (at 24.765 130.175) (size 0.6858) (drill 0.3302) (layers F.Cu B.Cu) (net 17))
 (segment (start 19.431 130.1135) (end 24.7035 130.1135) (width 0.254) (layer F.Cu) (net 17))
 (segment (start 24.765 130.175) (end 24.765 144.905) (width 0.254) (layer B.Cu) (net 17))
 (segment (start 24.765 144.905) (end 35.175 155.315) (width 0.254) (layer B.Cu) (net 17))
 (segment (start 8.235989 134.255011) (end 6.175999 136.315001) (width 0.254) (layer F.Cu) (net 18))
 (segment (start 6.175999 136.315001) (end 3.176 139.315) (width 0.254) (layer F.Cu) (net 18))
 (segment (start 8.235989 127.4546) (end 8.235989 134.255011) (width 0.254) (layer F.Cu) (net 18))
 (segment (start 8.23599 125.83951) (end 8.235989 127.4546) (width 0.254) (layer F.Cu) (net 18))
 (segment (start 11.582 122.4935) (end 8.23599 125.83951) (width 0.254) (layer F.Cu) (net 18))
 (segment (start 11.582 132.6535) (end 20.5135 132.6535) (width 0.254) (layer F.Cu) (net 19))
 (segment (start 20.5135 132.6535) (end 35.175 147.315) (width 0.254) (layer F.Cu) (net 19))
 (segment (start 11.582 119.9535) (end 3.176 128.3595) (width 0.254) (layer F.Cu) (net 20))
 (segment (start 3.176 128.3595) (end 3.176 131.315) (width 0.254) (layer F.Cu) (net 20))
 (segment (start 12.803314 102.1735) (end 11.582 102.1735) (width 0.254) (layer F.Cu) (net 10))
 (segment (start 13.645912 103.016098) (end 12.803314 102.1735) (width 0.254) (layer F.Cu) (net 10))
 (segment (start 24.758088 103.016098) (end 13.645912 103.016098) (width 0.254) (layer F.Cu) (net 10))
 (segment (start 25.600686 102.1735) (end 24.758088 103.016098) (width 0.254) (layer F.Cu) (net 10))
 (segment (start 26.822 102.1735) (end 25.600686 102.1735) (width 0.254) (layer F.Cu) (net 10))
 (segment (start 8.175001 78.314999) (end 11.175 75.315) (width 0.254) (layer B.Cu) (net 10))
 (segment (start 6.985 79.505) (end 8.175001 78.314999) (width 0.254) (layer B.Cu) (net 10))
 (segment (start 6.985 93.98) (end 6.985 79.505) (width 0.254) (layer B.Cu) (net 10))
 (segment (start 10.191399 97.186399) (end 6.985 93.98) (width 0.254) (layer F.Cu) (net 10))
 (via (at 6.985 93.98) (size 0.6858) (drill 0.3302) (layers F.Cu B.Cu) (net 10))
 (segment (start 11.582 102.1735) (end 10.191399 100.782899) (width 0.254) (layer F.Cu) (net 10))
 (segment (start 10.191399 100.782899) (end 10.191399 97.186399) (width 0.254) (layer F.Cu) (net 10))
 (segment (start 17.653 98.933) (end 17.818101 98.767899) (width 0.254) (layer F.Cu) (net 2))
 (segment (start 8.909011 90.5126) (end 15.89401 97.497599) (width 0.254) (layer F.Cu) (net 2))
 (segment (start 10.287 80.264) (end 8.909011 81.641989) (width 0.254) (layer F.Cu) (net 2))
 (segment (start 17.818101 98.767899) (end 18.161 98.425) (width 0.254) (layer F.Cu) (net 2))
 (segment (start 19.175 75.315) (end 14.226 80.264) (width 0.254) (layer F.Cu) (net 2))
 (segment (start 15.89401 97.497599) (end 15.89401 98.19001) (width 0.254) (layer F.Cu) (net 2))
 (segment (start 14.226 80.264) (end 10.287 80.264) (width 0.254) (layer F.Cu) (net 2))
 (segment (start 16.637 98.933) (end 17.653 98.933) (width 0.254) (layer F.Cu) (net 2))
 (segment (start 15.89401 98.19001) (end 16.637 98.933) (width 0.254) (layer F.Cu) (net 2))
 (segment (start 8.909011 81.641989) (end 8.909011 90.5126) (width 0.254) (layer F.Cu) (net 2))
 (segment (start 18.161 98.425) (end 22.86 103.124) (width 0.254) (layer B.Cu) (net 2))
 (segment (start 22.86 103.124) (end 22.86 121.285) (width 0.254) (layer B.Cu) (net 2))
 (via (at 18.161 98.425) (size 0.6858) (drill 0.3302) (layers F.Cu B.Cu) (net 2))
 (segment (start 22.86 132.715) (end 24.2205 132.715) (width 0.254) (layer F.Cu) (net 2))
 (segment (start 24.2205 132.715) (end 26.822 130.1135) (width 0.254) (layer F.Cu) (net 2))
 (segment (start 22.86 132.715) (end 22.86 131.445) (width 0.254) (layer B.Cu) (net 2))
 (segment (start 22.86 147.38736) (end 22.86 132.715) (width 0.254) (layer B.Cu) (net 2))
 (via (at 22.86 132.715) (size 0.6858) (drill 0.3302) (layers F.Cu B.Cu) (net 2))
 (segment (start 22.86 131.445) (end 22.86 121.285) (width 0.254) (layer B.Cu) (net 2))
 (segment (start 19.175 155.315) (end 19.175 151.07236) (width 0.254) (layer B.Cu) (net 2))
 (segment (start 19.175 151.07236) (end 22.86 147.38736) (width 0.254) (layer B.Cu) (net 2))
 (segment (start 25.4 86.36) (end 26.8224 86.36) (width 0.254) (layer B.Cu) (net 3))
 (segment (start 26.8224 86.36) (end 27.432 86.9696) (width 0.254) (layer B.Cu) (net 3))
 (segment (start 12.7 86.36) (end 15.24 86.36) (width 0.254) (layer F.Cu) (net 3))
 (segment (start 24.13 95.25) (end 24.13 104.902) (width 0.254) (layer B.Cu) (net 3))
 (segment (start 24.3185 104.7135) (end 24.13 104.902) (width 0.254) (layer B.Cu) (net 3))
 (segment (start 24.13 104.902) (end 24.13 124.8815) (width 0.254) (layer B.Cu) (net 3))
 (segment (start 26.822 104.7135) (end 24.3185 104.7135) (width 0.254) (layer B.Cu) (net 3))
 (segment (start 26.822 127.5735) (end 21.0165 127.5735) (width 0.254) (layer F.Cu) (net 3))
 (segment (start 21.0165 127.5735) (end 20.955 127.635) (width 0.254) (layer F.Cu) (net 3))
 (via (at 20.955 127.635) (size 0.6858) (drill 0.3302) (layers F.Cu B.Cu) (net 3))
 (segment (start 20.955 131.699) (end 20.955 131.445) (width 0.254) (layer B.Cu) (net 3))
 (segment (start 20.955 137.795) (end 20.955 131.699) (width 0.254) (layer B.Cu) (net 3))
 (segment (start 20.955 131.699) (end 20.955 127.635) (width 0.254) (layer B.Cu) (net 3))
 (segment (start 27.432 86.9696) (end 28.575 88.1126) (width 0.254) (layer B.Cu) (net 3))
 (segment (start 30.099 84.582) (end 29.614067 84.582) (width 0.254) (layer B.Cu) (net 3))
 (segment (start 29.614067 84.582) (end 27.432 86.764067) (width 0.254) (layer B.Cu) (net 3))
 (segment (start 27.432 86.764067) (end 27.432 86.9696) (width 0.254) (layer B.Cu) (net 3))
 (segment (start 30.48 83.947) (end 30.48 84.201) (width 0.254) (layer F.Cu) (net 3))
 (segment (start 30.48 84.201) (end 30.099 84.582) (width 0.254) (layer F.Cu) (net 3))
 (via (at 30.099 84.582) (size 0.6858) (drill 0.3302) (layers F.Cu B.Cu) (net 3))
 (segment (start 30.48 81.534) (end 30.48 83.947) (width 0.254) (layer F.Cu) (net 3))
 (segment (start 27.175 75.315) (end 30.48 78.62) (width 0.254) (layer B.Cu) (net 3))
 (segment (start 30.48 78.62) (end 30.48 81.534) (width 0.254) (layer B.Cu) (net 3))
 (via (at 30.48 81.534) (size 0.6858) (drill 0.3302) (layers F.Cu B.Cu) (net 3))
 (segment (start 25.4 86.36) (end 22.86 86.36) (width 0.254) (layer F.Cu) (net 3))
 (segment (start 22.86 86.36) (end 20.32 86.36) (width 0.254) (layer F.Cu) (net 3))
 (segment (start 20.32 86.36) (end 17.78 86.36) (width 0.254) (layer F.Cu) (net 3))
 (segment (start 15.24 86.36) (end 17.78 86.36) (width 0.254) (layer F.Cu) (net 3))
 (segment (start 26.822 127.5735) (end 30.5635 131.315) (width 0.254) (layer B.Cu) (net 3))
 (segment (start 30.5635 131.315) (end 35.175 131.315) (width 0.254) (layer B.Cu) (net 3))
 (segment (start 28.575 88.1126) (end 28.575 90.805) (width 0.254) (layer B.Cu) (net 3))
 (segment (start 28.575 90.805) (end 24.13 95.25) (width 0.254) (layer B.Cu) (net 3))
 (segment (start 24.13 124.8815) (end 26.822 127.5735) (width 0.254) (layer B.Cu) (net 3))
 (segment (start 11.175 138.05) (end 20.7 138.05) (width 0.254) (layer F.Cu) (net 3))
 (segment (start 20.7 138.05) (end 20.955 137.795) (width 0.254) (layer F.Cu) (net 3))
 (via (at 20.955 137.795) (size 0.6858) (drill 0.3302) (layers F.Cu B.Cu) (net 3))
 (via (at 11.175 138.05) (size 0.6858) (drill 0.3302) (layers F.Cu B.Cu) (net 3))
 (segment (start 11.175 141.225) (end 11.175 138.05) (width 0.254) (layer B.Cu) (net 3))
 (segment (start 11.175 155.315) (end 11.175 141.225) (width 0.254) (layer B.Cu) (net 3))
 (segment (start 25.4 83.82) (end 26.67 83.82) (width 0.254) (layer B.Cu) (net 9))
 (segment (start 26.67 83.82) (end 27.539901 84.689901) (width 0.254) (layer B.Cu) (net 9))
 (segment (start 28.581258 84.689901) (end 29.956159 83.315) (width 0.254) (layer B.Cu) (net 9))
 (segment (start 29.956159 83.315) (end 35.175 83.315) (width 0.254) (layer B.Cu) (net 9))
 (segment (start 27.539901 84.689901) (end 28.581258 84.689901) (width 0.254) (layer B.Cu) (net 9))
 (segment (start 31.647999 94.361) (end 31.647999 94.500543) (width 0.254) (layer B.Cu) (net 9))
 (segment (start 28.555994 99.789134) (end 28.55599 99.789134) (width 0.254) (layer B.Cu) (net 9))
 (segment (start 31.647999 86.842001) (end 31.647999 94.361) (width 0.254) (layer B.Cu) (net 9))
 (segment (start 31.647999 94.361) (end 31.647999 96.697129) (width 0.254) (layer B.Cu) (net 9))
 (segment (start 31.647999 96.697129) (end 28.555994 99.789134) (width 0.254) (layer B.Cu) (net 9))
 (segment (start 27.685599 111.469901) (end 26.822 112.3335) (width 0.254) (layer B.Cu) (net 9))
 (segment (start 35.175 83.315) (end 31.647999 86.842001) (width 0.254) (layer B.Cu) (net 9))
 (segment (start 28.55599 99.789134) (end 28.55599 110.59951) (width 0.254) (layer B.Cu) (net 9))
 (segment (start 28.55599 110.59951) (end 27.685599 111.469901) (width 0.254) (layer B.Cu) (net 9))
 (segment (start 27.685599 116.549901) (end 26.822 117.4135) (width 0.254) (layer B.Cu) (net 7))
 (segment (start 29.864011 114.371489) (end 27.685599 116.549901) (width 0.254) (layer B.Cu) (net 7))
 (segment (start 35.175 99.315) (end 29.864011 104.625989) (width 0.254) (layer B.Cu) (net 7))
 (segment (start 29.864011 104.625989) (end 29.864011 114.371489) (width 0.254) (layer B.Cu) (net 7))
 (segment (start 13.97 101.6) (end 13.97 122.6455) (width 0.254) (layer B.Cu) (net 23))
 (segment (start 13.97 122.6455) (end 11.582 125.0335) (width 0.254) (layer B.Cu) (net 23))
 (segment (start 13.97 96.498499) (end 13.97 101.6) (width 0.254) (layer F.Cu) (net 23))
 (via (at 13.97 101.6) (size 0.6858) (drill 0.3302) (layers F.Cu B.Cu) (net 23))
 (segment (start 8.255 80.645) (end 8.255 86.995) (width 0.254) (layer F.Cu) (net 23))
 (segment (start 8.255 86.995) (end 8.255 90.783499) (width 0.254) (layer F.Cu) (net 23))
 (segment (start 8.255 90.783499) (end 13.97 96.498499) (width 0.254) (layer F.Cu) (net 23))
 (segment (start 9.525 80.645) (end 8.255 80.645) (width 0.254) (layer B.Cu) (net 23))
 (via (at 8.255 80.645) (size 0.6858) (drill 0.3302) (layers F.Cu B.Cu) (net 23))
 (segment (start 18.2626 80.645) (end 9.525 80.645) (width 0.254) (layer B.Cu) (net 23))
 (segment (start 20.32 83.82) (end 20.32 82.7024) (width 0.254) (layer B.Cu) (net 23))
 (segment (start 20.32 82.7024) (end 18.2626 80.645) (width 0.254) (layer B.Cu) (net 23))
 (segment (start 8.89 127.7255) (end 8.89 141.601) (width 0.254) (layer F.Cu) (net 23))
 (segment (start 8.89 141.601) (end 3.176 147.315) (width 0.254) (layer F.Cu) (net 23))
 (segment (start 11.582 125.0335) (end 8.89 127.7255) (width 0.254) (layer F.Cu) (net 23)))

